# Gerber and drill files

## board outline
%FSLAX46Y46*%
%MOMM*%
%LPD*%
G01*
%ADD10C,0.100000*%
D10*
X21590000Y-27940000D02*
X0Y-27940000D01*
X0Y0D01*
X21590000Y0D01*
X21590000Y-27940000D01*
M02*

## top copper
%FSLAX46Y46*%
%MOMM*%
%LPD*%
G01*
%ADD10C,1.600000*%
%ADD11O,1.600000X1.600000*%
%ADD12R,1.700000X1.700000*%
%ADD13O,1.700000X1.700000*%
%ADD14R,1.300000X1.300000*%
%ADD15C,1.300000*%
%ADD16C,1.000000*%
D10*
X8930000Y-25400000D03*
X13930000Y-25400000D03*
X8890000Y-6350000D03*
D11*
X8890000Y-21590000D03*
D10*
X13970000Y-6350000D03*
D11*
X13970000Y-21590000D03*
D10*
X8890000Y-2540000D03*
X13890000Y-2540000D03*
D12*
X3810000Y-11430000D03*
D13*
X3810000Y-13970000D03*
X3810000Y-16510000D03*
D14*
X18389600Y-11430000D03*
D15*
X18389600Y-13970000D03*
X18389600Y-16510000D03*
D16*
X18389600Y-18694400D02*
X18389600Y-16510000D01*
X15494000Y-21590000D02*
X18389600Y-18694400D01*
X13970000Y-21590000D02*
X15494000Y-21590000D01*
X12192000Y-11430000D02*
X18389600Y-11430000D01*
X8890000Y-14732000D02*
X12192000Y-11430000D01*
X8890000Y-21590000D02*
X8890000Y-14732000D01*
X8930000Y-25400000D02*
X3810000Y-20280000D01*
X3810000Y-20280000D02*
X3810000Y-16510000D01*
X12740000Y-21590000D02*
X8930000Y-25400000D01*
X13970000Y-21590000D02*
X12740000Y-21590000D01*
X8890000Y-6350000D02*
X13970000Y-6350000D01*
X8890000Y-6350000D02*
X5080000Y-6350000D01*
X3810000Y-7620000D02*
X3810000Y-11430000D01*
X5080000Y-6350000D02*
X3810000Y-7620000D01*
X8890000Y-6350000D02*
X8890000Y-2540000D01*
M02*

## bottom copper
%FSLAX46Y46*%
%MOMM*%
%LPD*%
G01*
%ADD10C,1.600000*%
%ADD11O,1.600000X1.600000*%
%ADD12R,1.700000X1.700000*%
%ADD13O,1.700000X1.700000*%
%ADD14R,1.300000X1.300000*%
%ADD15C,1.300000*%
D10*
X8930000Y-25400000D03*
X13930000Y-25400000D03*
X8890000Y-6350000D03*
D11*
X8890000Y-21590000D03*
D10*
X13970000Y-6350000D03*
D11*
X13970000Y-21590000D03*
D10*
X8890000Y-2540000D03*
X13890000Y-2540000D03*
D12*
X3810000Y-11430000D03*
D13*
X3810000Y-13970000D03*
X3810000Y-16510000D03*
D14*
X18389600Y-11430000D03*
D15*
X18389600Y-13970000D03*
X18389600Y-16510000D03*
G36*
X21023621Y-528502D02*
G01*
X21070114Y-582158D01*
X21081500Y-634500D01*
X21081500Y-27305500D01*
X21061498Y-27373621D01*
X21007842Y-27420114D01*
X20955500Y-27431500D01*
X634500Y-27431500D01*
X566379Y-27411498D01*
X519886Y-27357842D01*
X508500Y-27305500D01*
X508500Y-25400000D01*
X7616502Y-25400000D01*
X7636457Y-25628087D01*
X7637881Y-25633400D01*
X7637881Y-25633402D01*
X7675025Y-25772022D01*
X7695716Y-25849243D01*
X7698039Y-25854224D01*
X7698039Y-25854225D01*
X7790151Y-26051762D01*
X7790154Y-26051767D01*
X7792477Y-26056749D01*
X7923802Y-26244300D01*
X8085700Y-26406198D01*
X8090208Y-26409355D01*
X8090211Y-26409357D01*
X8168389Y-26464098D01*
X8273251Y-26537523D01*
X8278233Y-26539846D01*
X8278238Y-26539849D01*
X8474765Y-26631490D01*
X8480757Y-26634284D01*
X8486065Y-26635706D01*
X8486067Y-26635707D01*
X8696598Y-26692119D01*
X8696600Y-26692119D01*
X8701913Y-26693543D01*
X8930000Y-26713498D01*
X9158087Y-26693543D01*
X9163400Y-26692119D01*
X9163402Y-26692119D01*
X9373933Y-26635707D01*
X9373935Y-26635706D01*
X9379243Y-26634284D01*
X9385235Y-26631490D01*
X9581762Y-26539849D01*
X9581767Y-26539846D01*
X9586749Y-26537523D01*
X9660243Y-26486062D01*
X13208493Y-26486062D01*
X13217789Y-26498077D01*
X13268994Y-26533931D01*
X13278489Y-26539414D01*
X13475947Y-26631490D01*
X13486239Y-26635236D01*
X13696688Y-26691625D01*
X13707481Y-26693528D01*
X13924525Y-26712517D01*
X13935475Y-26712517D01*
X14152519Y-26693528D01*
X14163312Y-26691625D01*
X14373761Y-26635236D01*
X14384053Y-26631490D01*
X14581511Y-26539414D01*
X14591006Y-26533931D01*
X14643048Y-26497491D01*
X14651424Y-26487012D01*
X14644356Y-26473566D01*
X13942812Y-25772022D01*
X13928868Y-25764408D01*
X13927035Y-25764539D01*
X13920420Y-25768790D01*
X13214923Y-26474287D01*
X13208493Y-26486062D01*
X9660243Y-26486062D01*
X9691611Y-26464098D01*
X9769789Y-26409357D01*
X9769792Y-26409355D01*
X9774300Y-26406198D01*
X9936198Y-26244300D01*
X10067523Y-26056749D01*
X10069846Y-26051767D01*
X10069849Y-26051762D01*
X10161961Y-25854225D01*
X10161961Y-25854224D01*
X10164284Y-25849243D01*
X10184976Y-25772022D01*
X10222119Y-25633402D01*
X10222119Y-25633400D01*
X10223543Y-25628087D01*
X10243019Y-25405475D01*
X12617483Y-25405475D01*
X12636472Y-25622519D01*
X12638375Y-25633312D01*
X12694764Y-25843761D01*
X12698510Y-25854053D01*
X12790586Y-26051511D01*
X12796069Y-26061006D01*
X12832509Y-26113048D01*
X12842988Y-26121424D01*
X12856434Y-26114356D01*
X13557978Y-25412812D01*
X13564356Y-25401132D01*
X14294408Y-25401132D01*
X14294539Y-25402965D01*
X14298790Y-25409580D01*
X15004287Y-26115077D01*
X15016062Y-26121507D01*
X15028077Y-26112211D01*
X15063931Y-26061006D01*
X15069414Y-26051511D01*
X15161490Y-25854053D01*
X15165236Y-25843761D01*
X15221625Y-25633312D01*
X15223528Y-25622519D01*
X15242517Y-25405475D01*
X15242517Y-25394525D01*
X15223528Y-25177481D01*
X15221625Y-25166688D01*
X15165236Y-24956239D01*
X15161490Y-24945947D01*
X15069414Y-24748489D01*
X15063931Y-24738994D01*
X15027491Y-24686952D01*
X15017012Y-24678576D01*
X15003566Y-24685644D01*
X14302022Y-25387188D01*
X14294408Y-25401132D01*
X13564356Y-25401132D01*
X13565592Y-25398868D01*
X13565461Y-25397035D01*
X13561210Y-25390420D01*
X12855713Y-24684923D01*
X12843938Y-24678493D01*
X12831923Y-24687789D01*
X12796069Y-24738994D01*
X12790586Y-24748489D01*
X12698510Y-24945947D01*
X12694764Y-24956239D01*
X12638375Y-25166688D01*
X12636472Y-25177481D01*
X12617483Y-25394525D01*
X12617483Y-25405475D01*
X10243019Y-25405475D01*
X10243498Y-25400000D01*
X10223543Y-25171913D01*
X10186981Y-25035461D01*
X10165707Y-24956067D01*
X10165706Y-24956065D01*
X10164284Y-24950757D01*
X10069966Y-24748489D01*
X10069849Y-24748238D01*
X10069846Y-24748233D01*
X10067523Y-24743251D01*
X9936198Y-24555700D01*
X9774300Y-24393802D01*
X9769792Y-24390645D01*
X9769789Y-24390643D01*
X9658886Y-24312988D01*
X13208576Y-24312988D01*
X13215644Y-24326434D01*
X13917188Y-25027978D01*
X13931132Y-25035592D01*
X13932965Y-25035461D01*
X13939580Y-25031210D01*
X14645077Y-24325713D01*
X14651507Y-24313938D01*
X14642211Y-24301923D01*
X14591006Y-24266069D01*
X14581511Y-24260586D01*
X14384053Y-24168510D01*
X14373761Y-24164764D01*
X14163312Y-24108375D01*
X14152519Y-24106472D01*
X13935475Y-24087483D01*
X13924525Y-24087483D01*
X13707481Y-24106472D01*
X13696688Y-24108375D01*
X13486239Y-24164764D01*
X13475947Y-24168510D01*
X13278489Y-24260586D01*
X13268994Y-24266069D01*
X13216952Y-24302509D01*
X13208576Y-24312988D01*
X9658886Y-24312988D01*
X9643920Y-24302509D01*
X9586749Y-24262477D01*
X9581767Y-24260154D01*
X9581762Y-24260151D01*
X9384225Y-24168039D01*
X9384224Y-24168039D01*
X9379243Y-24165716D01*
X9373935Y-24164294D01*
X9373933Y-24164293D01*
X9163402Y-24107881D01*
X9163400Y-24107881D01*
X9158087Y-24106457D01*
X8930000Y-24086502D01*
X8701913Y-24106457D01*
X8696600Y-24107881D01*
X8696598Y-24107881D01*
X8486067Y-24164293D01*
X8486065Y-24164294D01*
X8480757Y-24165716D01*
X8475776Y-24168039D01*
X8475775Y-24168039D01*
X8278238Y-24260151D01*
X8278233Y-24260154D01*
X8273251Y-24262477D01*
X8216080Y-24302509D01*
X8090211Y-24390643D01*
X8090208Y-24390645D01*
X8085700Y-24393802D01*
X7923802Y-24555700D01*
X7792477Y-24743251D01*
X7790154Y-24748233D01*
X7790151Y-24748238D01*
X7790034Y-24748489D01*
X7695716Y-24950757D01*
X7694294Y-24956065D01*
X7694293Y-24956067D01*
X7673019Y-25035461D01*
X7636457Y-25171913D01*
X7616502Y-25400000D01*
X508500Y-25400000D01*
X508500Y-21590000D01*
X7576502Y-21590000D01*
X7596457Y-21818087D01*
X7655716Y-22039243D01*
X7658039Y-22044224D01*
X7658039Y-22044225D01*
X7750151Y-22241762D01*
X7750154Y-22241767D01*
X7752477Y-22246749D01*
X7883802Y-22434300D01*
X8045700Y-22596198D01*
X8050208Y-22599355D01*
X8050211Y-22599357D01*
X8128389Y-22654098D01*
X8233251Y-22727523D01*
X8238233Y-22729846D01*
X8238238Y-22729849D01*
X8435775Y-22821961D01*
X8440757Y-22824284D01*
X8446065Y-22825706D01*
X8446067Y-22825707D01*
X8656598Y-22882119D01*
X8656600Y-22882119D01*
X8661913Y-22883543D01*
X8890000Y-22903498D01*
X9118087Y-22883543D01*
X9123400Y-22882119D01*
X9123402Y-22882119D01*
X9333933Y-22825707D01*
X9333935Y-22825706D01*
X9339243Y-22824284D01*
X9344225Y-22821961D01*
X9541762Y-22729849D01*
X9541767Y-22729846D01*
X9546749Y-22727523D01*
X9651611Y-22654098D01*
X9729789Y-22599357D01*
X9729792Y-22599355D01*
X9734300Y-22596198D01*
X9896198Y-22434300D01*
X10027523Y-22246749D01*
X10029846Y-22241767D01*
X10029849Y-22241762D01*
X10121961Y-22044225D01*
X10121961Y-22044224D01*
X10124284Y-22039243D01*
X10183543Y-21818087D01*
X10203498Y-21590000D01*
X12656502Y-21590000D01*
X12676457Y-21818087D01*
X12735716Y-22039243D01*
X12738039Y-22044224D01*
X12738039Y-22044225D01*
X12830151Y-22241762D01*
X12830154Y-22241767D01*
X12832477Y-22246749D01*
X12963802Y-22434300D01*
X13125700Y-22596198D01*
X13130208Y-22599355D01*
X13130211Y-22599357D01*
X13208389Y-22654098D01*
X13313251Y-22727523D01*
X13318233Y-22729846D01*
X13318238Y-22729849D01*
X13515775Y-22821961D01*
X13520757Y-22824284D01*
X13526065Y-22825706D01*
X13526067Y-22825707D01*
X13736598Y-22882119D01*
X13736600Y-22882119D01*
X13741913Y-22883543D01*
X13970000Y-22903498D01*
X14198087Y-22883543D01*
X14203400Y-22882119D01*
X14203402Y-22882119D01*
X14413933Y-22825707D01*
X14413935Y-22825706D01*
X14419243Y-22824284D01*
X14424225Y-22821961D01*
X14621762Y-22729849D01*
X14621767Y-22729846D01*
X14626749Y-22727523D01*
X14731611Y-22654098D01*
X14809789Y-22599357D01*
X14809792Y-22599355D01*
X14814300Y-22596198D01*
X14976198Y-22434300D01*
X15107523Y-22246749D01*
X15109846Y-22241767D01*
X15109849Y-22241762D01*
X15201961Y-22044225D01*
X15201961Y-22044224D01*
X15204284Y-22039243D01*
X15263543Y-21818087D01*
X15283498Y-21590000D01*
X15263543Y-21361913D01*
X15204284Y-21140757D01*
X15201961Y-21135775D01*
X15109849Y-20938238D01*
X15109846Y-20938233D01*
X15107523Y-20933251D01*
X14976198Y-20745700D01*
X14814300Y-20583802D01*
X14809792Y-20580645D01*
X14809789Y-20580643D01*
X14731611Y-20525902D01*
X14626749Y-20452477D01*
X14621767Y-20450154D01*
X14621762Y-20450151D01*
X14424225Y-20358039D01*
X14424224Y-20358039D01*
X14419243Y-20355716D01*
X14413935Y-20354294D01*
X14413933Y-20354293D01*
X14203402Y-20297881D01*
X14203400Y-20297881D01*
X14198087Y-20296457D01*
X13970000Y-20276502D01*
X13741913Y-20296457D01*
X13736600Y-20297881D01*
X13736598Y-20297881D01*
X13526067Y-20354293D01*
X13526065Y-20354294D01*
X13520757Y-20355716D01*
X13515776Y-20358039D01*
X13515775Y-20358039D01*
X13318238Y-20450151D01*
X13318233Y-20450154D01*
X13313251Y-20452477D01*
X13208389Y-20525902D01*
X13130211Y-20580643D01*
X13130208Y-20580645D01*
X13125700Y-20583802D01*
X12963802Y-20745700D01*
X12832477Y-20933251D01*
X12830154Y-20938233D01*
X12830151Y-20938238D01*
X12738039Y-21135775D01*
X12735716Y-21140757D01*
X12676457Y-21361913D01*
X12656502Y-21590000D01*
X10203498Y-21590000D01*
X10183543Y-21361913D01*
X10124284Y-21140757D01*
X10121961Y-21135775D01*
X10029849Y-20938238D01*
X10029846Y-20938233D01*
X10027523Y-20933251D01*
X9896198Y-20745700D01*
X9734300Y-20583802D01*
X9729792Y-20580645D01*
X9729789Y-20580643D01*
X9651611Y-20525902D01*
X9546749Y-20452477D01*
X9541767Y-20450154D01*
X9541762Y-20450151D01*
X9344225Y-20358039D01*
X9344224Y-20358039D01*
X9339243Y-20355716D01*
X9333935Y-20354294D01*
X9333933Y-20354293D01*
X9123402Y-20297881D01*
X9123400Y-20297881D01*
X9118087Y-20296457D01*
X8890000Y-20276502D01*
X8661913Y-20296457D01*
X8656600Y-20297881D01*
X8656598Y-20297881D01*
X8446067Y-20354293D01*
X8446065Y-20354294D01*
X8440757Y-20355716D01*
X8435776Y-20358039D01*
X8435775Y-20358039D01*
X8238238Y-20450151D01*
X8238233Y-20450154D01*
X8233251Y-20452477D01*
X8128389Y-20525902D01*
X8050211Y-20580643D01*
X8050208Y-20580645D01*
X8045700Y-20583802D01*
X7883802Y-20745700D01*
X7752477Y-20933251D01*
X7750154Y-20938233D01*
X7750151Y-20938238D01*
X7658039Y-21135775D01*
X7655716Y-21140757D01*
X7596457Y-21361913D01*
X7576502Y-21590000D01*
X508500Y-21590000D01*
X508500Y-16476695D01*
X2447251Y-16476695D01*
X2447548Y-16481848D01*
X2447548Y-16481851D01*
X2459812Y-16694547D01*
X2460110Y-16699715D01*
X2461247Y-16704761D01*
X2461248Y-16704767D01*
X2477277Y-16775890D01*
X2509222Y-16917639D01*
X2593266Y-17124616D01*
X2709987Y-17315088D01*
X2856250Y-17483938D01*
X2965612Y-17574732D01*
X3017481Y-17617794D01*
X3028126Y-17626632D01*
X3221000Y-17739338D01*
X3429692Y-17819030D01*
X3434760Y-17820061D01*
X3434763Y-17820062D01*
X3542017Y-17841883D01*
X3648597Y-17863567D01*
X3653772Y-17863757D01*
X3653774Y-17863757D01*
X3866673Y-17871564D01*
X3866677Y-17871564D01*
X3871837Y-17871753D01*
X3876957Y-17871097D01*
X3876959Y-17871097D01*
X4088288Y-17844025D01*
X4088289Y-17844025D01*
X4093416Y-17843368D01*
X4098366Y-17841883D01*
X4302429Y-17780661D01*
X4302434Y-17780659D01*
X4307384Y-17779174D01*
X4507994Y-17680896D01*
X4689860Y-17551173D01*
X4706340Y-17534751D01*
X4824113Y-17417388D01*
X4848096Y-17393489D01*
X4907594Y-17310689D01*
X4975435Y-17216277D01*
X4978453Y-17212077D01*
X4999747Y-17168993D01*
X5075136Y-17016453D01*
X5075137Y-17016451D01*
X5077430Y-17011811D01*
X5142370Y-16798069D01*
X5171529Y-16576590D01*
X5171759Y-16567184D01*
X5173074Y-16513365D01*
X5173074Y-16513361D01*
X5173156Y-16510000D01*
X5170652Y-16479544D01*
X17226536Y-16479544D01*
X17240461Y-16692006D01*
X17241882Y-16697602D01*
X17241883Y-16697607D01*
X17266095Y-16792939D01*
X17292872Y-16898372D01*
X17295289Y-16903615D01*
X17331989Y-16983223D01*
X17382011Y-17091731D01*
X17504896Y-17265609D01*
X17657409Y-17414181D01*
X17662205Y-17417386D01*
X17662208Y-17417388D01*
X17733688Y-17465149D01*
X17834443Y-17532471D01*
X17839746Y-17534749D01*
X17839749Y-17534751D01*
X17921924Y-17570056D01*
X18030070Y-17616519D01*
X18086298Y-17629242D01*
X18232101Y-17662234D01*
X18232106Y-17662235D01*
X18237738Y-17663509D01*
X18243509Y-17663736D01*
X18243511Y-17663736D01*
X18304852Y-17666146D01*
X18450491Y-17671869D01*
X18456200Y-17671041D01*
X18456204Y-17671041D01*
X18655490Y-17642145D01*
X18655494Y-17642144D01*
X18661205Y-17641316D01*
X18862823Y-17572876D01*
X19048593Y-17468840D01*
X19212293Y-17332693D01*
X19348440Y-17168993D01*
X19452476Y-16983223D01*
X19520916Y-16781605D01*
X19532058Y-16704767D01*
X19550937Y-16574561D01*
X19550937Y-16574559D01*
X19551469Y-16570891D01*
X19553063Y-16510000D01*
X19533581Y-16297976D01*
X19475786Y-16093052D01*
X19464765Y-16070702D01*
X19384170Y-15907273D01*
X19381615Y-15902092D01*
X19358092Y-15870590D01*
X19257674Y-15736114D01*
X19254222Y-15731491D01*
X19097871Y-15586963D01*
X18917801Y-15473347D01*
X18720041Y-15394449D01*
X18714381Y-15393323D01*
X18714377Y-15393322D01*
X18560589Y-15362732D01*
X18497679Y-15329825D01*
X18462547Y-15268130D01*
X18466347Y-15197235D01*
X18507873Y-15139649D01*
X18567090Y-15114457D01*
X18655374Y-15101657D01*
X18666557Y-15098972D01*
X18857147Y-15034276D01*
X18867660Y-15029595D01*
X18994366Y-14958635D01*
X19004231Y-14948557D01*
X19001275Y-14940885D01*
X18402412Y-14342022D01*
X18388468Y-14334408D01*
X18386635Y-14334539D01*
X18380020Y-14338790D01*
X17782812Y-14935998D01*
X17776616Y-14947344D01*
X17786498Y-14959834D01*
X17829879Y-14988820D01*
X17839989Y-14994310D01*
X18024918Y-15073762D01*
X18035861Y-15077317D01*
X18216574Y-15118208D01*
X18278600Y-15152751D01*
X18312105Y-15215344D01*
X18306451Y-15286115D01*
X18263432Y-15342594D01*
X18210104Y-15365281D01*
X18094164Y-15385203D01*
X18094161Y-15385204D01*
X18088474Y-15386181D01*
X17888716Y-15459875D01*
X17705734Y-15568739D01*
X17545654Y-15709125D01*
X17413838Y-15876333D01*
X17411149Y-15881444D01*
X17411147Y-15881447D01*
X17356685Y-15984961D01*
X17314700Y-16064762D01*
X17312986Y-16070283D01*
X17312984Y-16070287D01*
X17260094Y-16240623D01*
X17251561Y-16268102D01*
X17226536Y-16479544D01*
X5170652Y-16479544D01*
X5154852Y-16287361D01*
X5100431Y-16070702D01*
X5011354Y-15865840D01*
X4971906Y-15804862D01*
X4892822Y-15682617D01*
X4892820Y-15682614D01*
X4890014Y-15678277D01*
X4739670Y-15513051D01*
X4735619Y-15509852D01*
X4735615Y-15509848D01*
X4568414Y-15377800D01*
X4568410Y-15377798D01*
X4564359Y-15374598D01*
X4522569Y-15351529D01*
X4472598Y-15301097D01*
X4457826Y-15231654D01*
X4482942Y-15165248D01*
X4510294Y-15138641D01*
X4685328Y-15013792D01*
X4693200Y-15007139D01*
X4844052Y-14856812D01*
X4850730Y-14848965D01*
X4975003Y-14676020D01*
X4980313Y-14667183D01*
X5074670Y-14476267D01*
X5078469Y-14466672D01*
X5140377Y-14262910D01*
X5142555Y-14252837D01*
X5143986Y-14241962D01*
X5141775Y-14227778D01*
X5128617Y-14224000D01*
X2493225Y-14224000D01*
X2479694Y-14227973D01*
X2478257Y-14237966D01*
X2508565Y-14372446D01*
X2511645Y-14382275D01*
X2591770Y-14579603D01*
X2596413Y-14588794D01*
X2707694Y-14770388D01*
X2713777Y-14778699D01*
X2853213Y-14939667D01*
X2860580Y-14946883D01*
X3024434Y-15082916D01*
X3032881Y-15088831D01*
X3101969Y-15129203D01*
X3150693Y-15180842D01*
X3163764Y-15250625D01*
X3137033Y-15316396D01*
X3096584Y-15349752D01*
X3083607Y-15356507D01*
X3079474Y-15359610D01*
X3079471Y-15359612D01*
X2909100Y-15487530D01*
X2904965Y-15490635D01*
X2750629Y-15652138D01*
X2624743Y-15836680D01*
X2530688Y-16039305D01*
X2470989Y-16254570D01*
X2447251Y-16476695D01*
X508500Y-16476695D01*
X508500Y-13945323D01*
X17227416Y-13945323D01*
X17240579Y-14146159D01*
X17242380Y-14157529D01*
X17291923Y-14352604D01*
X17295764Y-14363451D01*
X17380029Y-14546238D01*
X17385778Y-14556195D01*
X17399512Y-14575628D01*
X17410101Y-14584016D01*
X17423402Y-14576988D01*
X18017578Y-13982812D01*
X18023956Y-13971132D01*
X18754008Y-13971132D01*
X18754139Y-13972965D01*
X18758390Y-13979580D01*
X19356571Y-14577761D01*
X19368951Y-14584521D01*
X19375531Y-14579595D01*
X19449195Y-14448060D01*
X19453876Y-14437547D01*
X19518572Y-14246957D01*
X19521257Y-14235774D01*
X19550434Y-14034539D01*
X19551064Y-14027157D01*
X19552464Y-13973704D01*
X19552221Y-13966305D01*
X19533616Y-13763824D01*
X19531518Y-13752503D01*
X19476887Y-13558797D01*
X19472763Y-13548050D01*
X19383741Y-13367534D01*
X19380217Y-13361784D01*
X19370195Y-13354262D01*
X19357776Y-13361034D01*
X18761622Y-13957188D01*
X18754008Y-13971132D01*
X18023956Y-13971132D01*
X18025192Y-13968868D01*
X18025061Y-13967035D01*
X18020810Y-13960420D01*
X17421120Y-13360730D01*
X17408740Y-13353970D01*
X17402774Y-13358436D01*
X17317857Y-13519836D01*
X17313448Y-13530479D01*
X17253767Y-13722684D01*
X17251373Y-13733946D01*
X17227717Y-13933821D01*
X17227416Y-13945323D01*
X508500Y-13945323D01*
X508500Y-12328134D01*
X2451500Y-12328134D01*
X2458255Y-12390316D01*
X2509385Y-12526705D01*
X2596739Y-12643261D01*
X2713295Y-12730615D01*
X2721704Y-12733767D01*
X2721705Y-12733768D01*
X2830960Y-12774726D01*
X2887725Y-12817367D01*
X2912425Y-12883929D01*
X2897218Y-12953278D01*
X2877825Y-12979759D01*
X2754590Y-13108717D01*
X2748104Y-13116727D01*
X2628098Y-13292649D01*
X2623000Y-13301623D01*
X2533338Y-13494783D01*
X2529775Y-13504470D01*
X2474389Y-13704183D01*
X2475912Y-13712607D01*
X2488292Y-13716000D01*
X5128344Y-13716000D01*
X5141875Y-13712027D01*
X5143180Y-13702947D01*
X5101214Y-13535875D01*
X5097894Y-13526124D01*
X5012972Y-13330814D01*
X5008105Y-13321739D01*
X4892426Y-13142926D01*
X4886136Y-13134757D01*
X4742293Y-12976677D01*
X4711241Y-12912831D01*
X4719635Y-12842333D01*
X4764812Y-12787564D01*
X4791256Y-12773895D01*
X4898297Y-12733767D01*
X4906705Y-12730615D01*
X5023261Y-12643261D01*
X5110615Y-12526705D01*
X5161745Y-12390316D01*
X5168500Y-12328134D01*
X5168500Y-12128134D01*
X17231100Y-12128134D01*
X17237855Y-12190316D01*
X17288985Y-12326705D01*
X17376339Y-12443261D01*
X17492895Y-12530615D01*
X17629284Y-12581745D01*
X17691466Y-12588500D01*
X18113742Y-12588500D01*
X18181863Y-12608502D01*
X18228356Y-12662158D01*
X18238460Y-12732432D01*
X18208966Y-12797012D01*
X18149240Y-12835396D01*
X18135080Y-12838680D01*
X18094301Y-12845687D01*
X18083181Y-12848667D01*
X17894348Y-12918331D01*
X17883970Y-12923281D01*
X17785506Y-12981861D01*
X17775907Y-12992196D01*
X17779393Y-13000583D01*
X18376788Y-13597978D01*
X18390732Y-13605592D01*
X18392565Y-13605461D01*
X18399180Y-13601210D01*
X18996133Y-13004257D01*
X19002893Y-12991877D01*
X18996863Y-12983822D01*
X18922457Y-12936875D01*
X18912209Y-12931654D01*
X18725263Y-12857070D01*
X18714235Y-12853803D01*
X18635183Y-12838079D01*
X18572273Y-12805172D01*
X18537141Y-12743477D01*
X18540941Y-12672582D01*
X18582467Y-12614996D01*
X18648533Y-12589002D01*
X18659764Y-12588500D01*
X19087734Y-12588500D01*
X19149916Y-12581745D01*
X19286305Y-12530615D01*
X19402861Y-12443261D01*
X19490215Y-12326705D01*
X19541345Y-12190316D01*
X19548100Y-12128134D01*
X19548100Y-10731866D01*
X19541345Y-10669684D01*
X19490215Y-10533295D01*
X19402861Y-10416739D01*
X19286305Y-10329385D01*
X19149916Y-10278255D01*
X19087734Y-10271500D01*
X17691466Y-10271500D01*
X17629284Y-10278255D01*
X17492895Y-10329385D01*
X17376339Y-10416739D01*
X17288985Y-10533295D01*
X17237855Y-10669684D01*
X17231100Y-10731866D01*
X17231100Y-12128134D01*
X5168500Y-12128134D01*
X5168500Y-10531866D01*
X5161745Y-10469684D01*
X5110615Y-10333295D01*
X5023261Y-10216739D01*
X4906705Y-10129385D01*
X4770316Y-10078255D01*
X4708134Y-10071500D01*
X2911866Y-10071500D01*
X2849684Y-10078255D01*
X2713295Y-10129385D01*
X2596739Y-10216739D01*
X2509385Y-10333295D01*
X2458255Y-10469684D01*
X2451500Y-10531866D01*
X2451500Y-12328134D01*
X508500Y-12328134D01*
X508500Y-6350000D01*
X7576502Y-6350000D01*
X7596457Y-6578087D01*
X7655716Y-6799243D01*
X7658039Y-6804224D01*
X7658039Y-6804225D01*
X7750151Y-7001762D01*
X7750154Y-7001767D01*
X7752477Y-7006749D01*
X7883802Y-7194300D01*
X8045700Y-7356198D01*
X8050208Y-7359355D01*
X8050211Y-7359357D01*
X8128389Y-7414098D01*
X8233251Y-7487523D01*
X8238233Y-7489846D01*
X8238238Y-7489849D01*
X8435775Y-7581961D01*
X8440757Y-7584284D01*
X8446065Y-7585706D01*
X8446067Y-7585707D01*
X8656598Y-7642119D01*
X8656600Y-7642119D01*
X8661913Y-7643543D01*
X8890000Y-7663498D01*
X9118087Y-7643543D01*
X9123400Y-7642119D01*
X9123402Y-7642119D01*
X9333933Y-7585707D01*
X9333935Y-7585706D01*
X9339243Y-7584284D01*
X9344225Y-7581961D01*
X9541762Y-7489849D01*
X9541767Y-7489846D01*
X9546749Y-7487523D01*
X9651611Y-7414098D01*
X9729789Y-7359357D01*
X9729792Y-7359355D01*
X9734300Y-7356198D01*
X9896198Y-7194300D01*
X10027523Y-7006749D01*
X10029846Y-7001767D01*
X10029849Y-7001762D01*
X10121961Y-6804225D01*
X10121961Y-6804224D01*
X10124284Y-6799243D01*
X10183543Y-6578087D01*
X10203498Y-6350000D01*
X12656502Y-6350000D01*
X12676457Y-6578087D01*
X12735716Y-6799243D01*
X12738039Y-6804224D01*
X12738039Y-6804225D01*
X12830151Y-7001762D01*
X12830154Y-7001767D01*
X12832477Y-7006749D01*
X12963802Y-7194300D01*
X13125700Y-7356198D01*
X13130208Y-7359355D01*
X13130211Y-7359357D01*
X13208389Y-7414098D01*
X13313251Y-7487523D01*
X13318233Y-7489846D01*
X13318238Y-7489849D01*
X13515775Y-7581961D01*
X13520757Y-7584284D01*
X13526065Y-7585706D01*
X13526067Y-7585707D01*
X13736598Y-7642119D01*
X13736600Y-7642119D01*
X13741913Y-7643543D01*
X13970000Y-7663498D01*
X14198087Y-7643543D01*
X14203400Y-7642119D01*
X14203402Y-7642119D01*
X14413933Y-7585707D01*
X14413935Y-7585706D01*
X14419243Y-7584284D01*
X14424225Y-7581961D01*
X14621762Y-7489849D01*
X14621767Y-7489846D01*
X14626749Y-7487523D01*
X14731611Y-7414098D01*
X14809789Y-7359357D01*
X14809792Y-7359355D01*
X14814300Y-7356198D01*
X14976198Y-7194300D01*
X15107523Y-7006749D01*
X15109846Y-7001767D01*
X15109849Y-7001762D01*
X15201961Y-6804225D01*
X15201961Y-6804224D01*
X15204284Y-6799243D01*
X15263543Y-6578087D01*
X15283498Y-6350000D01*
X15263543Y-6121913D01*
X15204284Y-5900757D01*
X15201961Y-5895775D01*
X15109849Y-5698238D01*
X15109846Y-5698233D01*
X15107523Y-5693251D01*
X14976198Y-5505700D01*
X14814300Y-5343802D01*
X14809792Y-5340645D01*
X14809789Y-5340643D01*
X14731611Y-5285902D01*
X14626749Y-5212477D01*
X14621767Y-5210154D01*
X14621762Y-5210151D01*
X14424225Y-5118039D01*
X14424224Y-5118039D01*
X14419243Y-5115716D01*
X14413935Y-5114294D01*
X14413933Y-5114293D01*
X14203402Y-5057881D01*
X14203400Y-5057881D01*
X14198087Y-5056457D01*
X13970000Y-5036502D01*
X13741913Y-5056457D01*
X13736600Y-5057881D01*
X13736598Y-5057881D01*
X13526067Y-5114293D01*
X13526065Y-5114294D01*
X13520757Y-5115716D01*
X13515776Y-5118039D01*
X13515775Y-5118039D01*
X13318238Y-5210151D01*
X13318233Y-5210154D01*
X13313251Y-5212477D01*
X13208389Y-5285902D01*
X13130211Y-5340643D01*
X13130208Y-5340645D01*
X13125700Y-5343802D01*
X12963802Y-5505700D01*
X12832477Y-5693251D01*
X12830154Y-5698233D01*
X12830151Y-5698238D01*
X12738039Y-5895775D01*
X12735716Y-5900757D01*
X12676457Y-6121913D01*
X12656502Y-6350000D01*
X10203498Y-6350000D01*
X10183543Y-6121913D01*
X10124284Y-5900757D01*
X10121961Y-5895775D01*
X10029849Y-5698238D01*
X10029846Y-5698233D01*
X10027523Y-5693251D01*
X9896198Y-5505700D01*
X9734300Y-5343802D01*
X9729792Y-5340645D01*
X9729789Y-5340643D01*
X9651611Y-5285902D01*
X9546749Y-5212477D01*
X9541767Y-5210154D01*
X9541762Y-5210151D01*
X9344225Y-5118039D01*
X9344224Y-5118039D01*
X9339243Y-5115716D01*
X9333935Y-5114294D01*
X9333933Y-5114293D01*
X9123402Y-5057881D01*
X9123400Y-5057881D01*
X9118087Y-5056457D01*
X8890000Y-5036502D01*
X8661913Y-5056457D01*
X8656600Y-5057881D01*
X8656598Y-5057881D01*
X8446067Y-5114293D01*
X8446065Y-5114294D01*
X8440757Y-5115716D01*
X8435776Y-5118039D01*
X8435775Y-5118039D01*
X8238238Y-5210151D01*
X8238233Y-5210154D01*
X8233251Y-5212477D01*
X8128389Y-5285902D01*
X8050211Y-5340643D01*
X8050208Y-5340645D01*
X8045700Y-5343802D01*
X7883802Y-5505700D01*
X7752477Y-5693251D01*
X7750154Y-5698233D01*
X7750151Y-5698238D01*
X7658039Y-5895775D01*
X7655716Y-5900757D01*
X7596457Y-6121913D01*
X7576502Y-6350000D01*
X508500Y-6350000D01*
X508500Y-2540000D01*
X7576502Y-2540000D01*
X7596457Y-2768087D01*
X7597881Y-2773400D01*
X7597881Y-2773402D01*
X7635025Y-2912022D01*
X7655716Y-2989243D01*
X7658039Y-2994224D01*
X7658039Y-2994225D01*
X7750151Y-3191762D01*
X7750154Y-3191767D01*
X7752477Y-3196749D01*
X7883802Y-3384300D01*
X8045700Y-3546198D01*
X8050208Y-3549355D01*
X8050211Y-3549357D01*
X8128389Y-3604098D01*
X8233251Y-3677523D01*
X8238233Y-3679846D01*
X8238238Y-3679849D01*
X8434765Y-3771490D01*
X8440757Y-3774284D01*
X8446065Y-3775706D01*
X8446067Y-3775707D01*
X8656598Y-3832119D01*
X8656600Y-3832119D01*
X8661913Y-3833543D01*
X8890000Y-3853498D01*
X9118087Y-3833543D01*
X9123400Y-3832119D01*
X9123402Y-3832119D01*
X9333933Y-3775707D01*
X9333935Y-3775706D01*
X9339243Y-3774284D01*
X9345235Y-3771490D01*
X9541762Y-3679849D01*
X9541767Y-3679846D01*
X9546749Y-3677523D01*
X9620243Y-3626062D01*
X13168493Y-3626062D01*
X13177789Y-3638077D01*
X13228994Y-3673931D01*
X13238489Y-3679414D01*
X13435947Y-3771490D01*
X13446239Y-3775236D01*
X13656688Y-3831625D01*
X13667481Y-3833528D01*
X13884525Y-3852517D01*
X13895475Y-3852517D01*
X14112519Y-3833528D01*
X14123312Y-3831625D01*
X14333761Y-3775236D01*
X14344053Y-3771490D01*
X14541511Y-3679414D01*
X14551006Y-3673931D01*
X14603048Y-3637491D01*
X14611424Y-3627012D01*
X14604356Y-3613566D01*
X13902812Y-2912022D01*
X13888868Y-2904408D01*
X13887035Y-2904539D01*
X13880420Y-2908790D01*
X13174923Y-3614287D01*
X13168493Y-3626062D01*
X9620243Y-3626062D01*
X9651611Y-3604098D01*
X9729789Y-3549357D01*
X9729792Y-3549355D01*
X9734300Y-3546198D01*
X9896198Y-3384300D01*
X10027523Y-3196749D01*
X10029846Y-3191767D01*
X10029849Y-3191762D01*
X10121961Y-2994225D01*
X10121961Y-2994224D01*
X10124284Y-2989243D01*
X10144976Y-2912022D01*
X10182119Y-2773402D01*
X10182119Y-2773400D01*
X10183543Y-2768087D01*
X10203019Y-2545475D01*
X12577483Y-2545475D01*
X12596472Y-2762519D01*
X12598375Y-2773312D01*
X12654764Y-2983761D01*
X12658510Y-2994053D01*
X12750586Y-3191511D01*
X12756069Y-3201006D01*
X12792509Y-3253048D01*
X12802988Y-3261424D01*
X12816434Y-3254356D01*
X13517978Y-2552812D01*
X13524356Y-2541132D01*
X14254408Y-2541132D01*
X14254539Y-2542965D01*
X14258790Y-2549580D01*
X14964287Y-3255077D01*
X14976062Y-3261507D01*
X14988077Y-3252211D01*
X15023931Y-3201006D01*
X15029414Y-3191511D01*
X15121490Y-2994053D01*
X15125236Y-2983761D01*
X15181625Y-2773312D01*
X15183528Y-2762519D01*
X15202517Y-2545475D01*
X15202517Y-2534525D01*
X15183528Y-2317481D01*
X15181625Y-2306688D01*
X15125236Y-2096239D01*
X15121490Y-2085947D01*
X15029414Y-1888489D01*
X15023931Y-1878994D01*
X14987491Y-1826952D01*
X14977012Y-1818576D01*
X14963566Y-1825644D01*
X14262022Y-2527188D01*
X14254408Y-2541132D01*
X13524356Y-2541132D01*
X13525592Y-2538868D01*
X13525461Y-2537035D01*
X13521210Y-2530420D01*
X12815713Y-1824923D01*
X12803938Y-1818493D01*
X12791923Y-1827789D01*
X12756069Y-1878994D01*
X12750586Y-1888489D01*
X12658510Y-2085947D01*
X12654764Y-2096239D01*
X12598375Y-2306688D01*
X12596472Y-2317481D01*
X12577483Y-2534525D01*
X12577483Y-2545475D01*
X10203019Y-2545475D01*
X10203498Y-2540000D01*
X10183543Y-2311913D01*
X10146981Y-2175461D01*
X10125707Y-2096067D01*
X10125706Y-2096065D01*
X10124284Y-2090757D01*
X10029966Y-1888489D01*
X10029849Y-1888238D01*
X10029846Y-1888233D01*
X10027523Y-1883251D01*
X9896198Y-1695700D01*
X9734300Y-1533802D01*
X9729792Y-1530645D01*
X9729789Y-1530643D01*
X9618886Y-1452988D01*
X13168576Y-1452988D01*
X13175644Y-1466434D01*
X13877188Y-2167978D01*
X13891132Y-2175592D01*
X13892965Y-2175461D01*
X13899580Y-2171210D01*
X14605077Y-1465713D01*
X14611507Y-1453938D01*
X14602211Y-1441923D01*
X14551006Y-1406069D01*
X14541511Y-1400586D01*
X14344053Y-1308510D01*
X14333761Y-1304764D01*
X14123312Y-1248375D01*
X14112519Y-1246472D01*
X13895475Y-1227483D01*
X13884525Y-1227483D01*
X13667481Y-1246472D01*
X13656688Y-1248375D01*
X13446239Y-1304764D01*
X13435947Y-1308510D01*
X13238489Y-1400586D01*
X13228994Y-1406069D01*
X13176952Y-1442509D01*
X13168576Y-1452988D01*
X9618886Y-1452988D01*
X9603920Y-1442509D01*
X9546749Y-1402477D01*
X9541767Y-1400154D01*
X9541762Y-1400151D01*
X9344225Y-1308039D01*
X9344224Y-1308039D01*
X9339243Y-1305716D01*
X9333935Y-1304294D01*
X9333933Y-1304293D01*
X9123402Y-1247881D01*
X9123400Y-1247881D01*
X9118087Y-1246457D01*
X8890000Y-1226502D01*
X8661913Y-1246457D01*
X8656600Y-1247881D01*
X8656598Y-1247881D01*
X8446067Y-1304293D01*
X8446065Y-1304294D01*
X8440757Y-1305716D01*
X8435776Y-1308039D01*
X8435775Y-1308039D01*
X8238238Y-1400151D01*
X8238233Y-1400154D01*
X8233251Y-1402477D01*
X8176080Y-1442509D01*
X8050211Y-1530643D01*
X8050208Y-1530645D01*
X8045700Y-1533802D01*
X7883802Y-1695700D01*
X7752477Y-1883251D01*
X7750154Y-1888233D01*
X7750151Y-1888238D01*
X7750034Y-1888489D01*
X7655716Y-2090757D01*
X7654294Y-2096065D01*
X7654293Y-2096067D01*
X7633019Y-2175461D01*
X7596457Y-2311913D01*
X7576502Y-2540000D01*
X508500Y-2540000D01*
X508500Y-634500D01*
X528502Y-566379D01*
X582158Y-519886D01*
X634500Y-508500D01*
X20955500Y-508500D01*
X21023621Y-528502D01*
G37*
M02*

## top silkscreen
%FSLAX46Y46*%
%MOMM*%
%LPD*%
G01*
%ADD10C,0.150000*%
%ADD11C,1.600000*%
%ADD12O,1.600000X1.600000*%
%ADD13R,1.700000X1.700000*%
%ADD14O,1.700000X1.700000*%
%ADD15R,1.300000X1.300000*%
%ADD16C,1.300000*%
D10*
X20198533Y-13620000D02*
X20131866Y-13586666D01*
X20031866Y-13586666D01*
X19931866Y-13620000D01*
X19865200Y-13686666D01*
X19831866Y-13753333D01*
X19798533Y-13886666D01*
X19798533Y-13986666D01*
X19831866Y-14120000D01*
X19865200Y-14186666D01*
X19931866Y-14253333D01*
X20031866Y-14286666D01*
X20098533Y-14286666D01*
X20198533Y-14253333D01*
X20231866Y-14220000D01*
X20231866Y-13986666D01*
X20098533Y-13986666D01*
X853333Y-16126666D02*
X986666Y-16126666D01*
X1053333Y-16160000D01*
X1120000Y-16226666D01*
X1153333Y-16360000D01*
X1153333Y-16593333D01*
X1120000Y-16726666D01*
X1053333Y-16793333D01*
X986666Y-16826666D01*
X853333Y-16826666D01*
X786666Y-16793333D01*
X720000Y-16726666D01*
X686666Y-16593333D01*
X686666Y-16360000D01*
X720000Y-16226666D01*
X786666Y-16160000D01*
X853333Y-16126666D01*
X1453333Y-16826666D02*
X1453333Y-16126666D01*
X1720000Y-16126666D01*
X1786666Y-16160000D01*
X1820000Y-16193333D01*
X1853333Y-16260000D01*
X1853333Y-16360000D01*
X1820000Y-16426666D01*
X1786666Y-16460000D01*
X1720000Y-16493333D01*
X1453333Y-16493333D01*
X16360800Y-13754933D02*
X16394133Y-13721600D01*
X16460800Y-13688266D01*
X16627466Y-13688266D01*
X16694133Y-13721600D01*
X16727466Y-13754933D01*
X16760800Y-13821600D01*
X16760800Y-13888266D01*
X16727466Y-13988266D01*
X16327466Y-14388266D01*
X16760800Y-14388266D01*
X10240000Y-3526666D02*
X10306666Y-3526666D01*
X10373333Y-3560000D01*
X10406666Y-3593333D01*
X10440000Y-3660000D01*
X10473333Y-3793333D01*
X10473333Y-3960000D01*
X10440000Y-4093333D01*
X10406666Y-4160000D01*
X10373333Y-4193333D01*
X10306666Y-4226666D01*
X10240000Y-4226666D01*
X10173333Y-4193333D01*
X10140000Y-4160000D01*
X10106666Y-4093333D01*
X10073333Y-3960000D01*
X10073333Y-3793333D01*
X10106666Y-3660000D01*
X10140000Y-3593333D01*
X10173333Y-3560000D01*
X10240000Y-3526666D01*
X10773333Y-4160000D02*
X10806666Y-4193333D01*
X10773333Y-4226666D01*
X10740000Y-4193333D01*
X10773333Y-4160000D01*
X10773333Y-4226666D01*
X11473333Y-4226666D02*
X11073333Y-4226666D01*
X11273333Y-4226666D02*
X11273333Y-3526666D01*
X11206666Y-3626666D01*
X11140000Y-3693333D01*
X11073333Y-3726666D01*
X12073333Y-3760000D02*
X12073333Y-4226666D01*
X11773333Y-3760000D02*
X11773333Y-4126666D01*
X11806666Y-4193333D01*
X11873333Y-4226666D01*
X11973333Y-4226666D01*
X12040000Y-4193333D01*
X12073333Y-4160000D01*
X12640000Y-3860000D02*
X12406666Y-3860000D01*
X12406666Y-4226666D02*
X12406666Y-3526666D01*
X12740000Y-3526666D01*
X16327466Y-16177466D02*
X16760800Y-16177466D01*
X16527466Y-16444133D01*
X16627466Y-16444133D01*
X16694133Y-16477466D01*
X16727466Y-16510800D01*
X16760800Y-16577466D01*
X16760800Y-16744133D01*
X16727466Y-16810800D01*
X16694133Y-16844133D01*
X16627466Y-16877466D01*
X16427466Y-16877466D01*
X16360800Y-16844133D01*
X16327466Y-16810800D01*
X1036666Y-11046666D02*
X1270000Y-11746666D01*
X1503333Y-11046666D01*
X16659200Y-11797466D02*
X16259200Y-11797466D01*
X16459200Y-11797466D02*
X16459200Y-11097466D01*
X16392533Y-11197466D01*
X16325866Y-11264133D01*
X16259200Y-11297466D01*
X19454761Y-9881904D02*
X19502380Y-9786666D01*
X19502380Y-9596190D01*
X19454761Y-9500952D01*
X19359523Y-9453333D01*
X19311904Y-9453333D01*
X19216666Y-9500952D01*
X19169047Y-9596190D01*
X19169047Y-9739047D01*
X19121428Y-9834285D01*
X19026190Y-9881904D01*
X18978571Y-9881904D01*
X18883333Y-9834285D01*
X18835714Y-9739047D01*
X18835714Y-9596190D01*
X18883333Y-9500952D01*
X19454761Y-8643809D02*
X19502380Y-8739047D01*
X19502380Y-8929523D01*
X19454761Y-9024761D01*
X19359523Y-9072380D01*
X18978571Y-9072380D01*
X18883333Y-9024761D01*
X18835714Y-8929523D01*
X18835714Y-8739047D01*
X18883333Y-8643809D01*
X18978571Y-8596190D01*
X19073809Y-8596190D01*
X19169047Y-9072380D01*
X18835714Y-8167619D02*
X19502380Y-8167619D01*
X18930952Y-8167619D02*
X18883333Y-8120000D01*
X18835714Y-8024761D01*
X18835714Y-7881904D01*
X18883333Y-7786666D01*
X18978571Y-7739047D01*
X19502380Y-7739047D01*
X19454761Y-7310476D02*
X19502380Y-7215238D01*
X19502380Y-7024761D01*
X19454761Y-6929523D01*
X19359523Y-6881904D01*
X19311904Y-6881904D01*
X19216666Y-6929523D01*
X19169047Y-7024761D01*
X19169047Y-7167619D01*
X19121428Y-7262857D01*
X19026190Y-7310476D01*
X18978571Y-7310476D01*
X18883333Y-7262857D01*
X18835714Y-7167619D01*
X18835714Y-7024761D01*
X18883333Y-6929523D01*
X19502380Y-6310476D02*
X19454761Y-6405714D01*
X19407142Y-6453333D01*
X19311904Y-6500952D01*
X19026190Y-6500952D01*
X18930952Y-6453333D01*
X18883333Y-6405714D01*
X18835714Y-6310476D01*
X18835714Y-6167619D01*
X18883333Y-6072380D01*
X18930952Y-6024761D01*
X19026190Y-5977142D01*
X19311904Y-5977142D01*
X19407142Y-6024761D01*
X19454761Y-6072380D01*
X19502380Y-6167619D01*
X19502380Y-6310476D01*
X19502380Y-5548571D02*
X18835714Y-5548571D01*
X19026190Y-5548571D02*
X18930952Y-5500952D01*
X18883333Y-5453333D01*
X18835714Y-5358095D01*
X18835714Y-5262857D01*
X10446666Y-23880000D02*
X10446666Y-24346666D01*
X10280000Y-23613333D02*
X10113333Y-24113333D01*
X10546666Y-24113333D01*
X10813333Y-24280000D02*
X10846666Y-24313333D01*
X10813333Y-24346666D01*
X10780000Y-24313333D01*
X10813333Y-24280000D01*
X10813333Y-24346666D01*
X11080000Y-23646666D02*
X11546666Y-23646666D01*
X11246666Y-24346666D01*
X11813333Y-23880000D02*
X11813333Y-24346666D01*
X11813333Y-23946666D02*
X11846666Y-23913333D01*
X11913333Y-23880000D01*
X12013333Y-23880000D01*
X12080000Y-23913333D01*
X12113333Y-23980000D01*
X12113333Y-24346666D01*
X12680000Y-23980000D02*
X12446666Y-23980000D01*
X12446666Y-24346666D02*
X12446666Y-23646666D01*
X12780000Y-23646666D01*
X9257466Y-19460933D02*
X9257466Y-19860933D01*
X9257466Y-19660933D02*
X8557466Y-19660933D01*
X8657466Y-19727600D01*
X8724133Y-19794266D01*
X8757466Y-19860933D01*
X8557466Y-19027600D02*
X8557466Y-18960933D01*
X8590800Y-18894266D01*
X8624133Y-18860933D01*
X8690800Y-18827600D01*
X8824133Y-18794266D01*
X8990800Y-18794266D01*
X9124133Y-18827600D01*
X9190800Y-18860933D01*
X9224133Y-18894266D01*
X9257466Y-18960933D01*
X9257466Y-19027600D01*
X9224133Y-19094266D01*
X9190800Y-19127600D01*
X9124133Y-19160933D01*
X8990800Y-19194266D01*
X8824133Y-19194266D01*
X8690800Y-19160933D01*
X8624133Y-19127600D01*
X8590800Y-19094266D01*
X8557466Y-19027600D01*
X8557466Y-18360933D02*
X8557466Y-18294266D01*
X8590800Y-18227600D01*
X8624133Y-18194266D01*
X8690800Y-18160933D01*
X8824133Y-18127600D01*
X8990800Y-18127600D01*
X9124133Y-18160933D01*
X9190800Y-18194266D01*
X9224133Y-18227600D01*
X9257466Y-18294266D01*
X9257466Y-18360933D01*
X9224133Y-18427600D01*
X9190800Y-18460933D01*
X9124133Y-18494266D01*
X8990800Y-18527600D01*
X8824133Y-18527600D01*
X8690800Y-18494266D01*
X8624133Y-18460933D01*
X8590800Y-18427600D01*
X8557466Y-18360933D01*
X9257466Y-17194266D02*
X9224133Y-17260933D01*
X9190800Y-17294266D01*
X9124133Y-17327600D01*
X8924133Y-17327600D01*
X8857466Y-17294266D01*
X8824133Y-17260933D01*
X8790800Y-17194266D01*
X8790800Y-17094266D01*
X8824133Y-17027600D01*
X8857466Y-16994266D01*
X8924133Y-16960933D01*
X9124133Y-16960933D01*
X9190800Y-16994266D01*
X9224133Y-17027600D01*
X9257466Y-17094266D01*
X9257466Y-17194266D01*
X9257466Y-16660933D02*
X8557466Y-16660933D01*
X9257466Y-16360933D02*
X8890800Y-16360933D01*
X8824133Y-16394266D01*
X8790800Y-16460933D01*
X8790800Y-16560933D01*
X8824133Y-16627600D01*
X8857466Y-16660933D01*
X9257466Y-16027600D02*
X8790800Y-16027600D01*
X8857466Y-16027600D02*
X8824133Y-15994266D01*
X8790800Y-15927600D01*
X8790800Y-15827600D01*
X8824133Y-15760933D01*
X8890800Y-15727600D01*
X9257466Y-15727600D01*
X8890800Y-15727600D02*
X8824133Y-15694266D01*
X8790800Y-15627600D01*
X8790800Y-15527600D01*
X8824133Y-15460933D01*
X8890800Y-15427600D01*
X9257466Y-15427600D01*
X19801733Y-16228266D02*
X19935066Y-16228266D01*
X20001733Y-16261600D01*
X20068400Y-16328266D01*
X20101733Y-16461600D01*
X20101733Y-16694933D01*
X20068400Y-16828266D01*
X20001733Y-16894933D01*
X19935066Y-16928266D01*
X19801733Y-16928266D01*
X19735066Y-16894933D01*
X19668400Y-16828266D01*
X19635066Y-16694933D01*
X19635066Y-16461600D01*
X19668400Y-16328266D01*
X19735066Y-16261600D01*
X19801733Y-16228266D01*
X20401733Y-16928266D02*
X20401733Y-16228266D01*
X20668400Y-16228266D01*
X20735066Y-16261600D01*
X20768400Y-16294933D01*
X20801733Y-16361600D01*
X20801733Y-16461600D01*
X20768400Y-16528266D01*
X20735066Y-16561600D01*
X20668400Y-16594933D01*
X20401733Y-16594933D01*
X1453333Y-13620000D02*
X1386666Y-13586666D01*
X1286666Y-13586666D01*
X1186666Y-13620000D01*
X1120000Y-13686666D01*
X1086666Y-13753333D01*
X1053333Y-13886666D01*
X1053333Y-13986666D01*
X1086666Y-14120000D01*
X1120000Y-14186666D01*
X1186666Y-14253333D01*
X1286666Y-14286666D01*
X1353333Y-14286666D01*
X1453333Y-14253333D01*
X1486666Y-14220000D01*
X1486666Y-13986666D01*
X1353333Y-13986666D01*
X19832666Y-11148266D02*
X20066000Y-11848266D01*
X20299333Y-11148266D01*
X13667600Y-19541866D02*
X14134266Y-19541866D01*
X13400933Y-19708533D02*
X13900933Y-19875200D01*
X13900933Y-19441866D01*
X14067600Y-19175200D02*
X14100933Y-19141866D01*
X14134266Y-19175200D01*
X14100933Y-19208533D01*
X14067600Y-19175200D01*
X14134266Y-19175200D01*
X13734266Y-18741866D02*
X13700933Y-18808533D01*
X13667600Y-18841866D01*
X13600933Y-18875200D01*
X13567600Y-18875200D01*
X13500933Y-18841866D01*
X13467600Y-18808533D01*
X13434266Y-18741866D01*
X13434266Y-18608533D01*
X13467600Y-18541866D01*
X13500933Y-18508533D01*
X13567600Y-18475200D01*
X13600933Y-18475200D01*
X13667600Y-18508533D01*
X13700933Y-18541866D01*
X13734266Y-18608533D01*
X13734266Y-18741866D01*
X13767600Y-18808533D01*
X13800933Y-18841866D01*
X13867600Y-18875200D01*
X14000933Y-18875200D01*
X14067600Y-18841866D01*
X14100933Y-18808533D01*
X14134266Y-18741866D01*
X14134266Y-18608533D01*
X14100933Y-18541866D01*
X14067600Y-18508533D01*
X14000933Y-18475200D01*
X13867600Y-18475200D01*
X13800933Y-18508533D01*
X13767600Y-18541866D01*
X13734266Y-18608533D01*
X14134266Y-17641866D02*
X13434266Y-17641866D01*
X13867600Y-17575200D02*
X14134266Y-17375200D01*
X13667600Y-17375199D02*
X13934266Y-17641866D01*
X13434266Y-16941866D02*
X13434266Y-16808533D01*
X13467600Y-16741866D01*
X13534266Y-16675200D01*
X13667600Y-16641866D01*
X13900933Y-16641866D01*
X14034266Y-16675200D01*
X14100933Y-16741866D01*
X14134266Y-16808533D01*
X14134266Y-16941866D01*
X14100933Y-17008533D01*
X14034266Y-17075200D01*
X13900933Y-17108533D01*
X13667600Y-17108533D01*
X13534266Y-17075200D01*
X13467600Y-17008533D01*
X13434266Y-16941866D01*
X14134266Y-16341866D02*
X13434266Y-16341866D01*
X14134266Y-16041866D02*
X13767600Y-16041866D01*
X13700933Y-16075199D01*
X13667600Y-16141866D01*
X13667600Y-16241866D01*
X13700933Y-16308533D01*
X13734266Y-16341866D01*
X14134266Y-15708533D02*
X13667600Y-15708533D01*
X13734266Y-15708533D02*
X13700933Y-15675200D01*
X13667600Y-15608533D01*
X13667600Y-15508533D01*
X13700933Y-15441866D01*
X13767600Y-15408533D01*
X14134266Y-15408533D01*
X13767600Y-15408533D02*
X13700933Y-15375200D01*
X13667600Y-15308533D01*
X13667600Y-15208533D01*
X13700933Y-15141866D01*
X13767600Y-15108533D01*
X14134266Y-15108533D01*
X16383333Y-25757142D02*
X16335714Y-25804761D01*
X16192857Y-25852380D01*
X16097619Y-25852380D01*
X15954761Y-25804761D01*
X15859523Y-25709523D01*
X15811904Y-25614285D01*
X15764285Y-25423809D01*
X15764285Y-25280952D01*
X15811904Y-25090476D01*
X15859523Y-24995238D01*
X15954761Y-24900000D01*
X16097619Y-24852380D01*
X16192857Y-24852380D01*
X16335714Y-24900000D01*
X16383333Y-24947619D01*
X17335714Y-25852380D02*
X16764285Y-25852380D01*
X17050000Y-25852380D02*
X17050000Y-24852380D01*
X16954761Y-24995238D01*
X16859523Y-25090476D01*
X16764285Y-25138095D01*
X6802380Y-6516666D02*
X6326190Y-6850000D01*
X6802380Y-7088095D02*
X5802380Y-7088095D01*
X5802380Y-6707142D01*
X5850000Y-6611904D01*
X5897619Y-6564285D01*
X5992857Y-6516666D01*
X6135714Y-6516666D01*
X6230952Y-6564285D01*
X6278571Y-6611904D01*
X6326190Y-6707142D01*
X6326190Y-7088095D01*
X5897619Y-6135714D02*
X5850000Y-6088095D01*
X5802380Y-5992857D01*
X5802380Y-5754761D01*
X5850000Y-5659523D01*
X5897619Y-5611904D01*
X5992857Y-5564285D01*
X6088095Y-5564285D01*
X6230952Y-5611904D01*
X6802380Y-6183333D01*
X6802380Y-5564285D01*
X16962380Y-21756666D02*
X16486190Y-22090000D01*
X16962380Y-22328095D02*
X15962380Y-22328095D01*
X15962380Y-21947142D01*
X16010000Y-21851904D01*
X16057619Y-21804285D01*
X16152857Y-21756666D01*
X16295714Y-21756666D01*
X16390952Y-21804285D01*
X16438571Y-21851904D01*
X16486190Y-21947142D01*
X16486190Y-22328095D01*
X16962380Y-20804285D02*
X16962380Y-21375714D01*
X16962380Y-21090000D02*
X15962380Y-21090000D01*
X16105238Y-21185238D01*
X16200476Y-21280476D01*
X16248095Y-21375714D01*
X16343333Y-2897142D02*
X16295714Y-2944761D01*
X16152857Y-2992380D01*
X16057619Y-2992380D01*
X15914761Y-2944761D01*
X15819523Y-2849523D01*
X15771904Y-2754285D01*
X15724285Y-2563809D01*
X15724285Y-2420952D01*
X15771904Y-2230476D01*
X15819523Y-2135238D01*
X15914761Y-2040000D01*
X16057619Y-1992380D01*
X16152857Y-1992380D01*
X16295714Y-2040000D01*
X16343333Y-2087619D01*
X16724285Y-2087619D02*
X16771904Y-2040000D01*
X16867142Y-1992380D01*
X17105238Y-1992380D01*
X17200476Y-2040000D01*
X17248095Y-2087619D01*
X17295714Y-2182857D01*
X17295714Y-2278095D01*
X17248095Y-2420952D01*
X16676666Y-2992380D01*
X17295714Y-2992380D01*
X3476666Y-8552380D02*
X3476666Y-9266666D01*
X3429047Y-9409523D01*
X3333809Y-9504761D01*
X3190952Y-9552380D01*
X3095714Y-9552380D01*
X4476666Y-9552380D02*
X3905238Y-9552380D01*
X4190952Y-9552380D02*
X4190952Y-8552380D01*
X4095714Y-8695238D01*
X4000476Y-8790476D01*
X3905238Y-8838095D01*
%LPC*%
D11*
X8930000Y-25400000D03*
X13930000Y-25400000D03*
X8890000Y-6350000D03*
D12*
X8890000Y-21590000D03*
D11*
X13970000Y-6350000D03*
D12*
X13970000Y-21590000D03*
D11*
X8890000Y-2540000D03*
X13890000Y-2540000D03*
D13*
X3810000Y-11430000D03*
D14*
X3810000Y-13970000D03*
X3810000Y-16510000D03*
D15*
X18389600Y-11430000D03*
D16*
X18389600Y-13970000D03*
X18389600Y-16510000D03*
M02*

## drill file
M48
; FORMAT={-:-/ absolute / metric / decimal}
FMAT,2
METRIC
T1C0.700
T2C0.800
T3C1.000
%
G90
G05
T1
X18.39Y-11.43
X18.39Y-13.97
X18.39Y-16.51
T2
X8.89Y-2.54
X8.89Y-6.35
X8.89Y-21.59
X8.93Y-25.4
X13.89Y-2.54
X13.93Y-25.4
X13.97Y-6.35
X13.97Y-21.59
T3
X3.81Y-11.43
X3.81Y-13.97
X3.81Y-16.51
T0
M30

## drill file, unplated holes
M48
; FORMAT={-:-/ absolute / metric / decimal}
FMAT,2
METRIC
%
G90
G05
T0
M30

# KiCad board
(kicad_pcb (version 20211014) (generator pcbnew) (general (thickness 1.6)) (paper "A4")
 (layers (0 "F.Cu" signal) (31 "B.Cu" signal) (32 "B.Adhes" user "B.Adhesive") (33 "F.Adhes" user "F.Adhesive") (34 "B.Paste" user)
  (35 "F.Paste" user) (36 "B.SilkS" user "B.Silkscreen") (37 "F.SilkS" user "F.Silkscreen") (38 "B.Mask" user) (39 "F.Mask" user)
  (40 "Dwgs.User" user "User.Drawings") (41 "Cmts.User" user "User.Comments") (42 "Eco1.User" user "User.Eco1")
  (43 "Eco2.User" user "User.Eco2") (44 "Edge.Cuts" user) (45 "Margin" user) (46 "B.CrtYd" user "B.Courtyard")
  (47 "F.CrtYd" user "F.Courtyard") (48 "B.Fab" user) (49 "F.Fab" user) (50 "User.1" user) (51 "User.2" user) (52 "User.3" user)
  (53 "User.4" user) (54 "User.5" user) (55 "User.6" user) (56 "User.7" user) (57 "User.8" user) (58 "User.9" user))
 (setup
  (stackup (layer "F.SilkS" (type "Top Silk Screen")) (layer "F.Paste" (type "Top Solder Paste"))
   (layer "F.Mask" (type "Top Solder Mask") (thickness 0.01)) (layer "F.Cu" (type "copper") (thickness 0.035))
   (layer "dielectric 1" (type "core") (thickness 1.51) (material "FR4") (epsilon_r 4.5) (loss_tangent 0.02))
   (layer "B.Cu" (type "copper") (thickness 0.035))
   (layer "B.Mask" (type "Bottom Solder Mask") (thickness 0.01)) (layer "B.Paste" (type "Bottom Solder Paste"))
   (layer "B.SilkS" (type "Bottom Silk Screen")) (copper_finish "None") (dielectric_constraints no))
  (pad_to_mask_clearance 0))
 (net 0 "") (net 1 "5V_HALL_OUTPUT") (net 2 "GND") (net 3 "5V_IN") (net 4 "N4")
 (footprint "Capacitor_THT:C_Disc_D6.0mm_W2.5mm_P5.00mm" (layer "F.Cu") (at 8.93 25.4)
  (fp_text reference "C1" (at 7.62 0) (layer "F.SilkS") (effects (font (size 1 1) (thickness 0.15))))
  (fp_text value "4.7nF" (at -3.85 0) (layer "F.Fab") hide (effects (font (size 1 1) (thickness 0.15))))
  (pad "1" thru_hole circle (at 0 0) (size 1.6 1.6) (drill 0.8) (layers *.Cu *.Mask) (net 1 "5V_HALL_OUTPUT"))
  (pad "2" thru_hole circle (at 5 0) (size 1.6 1.6) (drill 0.8) (layers *.Cu *.Mask) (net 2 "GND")))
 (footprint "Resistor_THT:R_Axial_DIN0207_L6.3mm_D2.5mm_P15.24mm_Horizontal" (layer "F.Cu") (at 8.89 6.35 -90)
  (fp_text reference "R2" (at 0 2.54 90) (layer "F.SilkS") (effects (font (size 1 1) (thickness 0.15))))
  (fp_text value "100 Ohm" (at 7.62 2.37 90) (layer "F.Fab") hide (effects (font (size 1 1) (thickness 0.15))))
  (pad "1" thru_hole circle (at 0 0 270) (size 1.6 1.6) (drill 0.8) (layers *.Cu *.Mask) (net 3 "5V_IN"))
  (pad "2" thru_hole oval (at 15.24 0 270) (size 1.6 1.6) (drill 0.8) (layers *.Cu *.Mask) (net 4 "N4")))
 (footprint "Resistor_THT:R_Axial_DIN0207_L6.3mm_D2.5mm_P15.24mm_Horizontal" (layer "F.Cu") (at 13.97 6.35 -90)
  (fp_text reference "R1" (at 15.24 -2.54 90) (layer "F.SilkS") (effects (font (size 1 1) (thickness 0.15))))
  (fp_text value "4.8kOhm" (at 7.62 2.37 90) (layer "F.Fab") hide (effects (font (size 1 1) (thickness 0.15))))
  (pad "1" thru_hole circle (at 0 0 270) (size 1.6 1.6) (drill 0.8) (layers *.Cu *.Mask) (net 3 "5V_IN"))
  (pad "2" thru_hole oval (at 15.24 0 270) (size 1.6 1.6) (drill 0.8) (layers *.Cu *.Mask) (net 1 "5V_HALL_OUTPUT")))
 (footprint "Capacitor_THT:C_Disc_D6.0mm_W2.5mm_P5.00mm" (layer "F.Cu") (at 8.89 2.54)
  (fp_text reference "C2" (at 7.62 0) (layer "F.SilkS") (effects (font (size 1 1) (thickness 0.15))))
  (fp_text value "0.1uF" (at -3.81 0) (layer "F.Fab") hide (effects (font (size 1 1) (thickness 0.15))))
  (pad "1" thru_hole circle (at 0 0) (size 1.6 1.6) (drill 0.8) (layers *.Cu *.Mask) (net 3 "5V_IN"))
  (pad "2" thru_hole circle (at 5 0) (size 1.6 1.6) (drill 0.8) (layers *.Cu *.Mask) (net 2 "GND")))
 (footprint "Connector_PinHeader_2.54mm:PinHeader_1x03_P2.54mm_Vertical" (layer "F.Cu") (at 3.81 11.43)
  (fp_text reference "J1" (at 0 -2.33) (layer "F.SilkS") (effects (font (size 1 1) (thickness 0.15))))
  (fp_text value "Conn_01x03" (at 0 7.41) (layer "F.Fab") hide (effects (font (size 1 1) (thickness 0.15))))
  (pad "1" thru_hole rect (at 0 0) (size 1.7 1.7) (drill 1) (layers *.Cu *.Mask) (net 3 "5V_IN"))
  (pad "2" thru_hole oval (at 0 2.54) (size 1.7 1.7) (drill 1) (layers *.Cu *.Mask) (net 2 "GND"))
  (pad "3" thru_hole oval (at 0 5.08) (size 1.7 1.7) (drill 1) (layers *.Cu *.Mask) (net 1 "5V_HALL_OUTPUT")))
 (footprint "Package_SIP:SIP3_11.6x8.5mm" (layer "F.Cu") (at 18.3896 11.43 -90)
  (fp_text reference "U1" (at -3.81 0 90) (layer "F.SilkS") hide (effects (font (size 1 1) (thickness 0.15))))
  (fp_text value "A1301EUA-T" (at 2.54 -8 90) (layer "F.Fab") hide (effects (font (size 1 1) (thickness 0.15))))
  (pad "1" thru_hole rect (at 0 0 180) (size 1.3 1.3) (drill 0.7) (layers *.Cu *.Mask) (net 4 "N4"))
  (pad "2" thru_hole circle (at 2.54 0 90) (size 1.3 1.3) (drill 0.7) (layers *.Cu *.Mask) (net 2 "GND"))
  (pad "3" thru_hole circle (at 5.08 0 180) (size 1.3 1.3) (drill 0.7) (layers *.Cu *.Mask) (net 1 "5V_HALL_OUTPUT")))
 (gr_poly (pts (xy 21.59 27.94) (xy 0 27.94) (xy 0 0) (xy 21.59 0)) (layer "Edge.Cuts") (width 0.1) (fill none))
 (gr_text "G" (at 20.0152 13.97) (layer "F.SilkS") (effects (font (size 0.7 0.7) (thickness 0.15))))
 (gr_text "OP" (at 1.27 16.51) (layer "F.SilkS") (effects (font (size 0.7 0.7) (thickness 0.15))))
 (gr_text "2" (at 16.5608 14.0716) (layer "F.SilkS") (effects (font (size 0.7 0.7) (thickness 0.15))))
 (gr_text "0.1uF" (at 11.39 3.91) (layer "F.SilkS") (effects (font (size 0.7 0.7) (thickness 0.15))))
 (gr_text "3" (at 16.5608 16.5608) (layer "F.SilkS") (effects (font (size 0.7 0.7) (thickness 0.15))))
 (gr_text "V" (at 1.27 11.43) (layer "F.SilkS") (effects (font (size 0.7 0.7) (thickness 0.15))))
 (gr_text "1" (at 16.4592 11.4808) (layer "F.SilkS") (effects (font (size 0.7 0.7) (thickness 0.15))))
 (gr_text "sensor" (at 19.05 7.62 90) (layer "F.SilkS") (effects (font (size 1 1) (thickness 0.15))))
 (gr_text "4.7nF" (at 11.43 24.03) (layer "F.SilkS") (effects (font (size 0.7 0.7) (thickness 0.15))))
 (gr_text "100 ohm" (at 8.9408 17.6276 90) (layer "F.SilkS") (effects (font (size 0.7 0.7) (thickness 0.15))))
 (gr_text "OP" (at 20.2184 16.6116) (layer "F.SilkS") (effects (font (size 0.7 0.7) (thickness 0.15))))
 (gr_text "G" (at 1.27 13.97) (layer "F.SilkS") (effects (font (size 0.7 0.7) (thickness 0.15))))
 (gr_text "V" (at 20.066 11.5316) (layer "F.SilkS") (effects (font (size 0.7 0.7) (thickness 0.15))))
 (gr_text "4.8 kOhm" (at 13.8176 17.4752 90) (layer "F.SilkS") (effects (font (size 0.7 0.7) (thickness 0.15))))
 (segment (start 8.93 25.4) (end 3.81 20.28) (width 1) (layer "F.Cu") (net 1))
 (segment (start 3.81 20.28) (end 3.81 16.51) (width 1) (layer "F.Cu") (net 1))
 (segment (start 12.74 21.59) (end 8.93 25.4) (width 1) (layer "F.Cu") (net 1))
 (segment (start 18.3896 18.6944) (end 18.3896 16.51) (width 1) (layer "F.Cu") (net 1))
 (segment (start 13.97 21.59) (end 12.74 21.59) (width 1) (layer "F.Cu") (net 1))
 (segment (start 15.494 21.59) (end 18.3896 18.6944) (width 1) (layer "F.Cu") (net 1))
 (segment (start 13.97 21.59) (end 15.494 21.59) (width 1) (layer "F.Cu") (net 1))
 (segment (start 8.89 6.35) (end 13.97 6.35) (width 1) (layer "F.Cu") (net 3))
 (segment (start 8.89 6.35) (end 5.08 6.35) (width 1) (layer "F.Cu") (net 3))
 (segment (start 3.81 7.62) (end 3.81 11.43) (width 1) (layer "F.Cu") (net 3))
 (segment (start 5.08 6.35) (end 3.81 7.62) (width 1) (layer "F.Cu") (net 3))
 (segment (start 8.89 6.35) (end 8.89 2.54) (width 1) (layer "F.Cu") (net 3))
 (segment (start 8.89 14.732) (end 12.192 11.43) (width 1) (layer "F.Cu") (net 4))
 (segment (start 8.89 21.59) (end 8.89 14.732) (width 1) (layer "F.Cu") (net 4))
 (segment (start 12.192 11.43) (end 18.3896 11.43) (width 1) (layer "F.Cu") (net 4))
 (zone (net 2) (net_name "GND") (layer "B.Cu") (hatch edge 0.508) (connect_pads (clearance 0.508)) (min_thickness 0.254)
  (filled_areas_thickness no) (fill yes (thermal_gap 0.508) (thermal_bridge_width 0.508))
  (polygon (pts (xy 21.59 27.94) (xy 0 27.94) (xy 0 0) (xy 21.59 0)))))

